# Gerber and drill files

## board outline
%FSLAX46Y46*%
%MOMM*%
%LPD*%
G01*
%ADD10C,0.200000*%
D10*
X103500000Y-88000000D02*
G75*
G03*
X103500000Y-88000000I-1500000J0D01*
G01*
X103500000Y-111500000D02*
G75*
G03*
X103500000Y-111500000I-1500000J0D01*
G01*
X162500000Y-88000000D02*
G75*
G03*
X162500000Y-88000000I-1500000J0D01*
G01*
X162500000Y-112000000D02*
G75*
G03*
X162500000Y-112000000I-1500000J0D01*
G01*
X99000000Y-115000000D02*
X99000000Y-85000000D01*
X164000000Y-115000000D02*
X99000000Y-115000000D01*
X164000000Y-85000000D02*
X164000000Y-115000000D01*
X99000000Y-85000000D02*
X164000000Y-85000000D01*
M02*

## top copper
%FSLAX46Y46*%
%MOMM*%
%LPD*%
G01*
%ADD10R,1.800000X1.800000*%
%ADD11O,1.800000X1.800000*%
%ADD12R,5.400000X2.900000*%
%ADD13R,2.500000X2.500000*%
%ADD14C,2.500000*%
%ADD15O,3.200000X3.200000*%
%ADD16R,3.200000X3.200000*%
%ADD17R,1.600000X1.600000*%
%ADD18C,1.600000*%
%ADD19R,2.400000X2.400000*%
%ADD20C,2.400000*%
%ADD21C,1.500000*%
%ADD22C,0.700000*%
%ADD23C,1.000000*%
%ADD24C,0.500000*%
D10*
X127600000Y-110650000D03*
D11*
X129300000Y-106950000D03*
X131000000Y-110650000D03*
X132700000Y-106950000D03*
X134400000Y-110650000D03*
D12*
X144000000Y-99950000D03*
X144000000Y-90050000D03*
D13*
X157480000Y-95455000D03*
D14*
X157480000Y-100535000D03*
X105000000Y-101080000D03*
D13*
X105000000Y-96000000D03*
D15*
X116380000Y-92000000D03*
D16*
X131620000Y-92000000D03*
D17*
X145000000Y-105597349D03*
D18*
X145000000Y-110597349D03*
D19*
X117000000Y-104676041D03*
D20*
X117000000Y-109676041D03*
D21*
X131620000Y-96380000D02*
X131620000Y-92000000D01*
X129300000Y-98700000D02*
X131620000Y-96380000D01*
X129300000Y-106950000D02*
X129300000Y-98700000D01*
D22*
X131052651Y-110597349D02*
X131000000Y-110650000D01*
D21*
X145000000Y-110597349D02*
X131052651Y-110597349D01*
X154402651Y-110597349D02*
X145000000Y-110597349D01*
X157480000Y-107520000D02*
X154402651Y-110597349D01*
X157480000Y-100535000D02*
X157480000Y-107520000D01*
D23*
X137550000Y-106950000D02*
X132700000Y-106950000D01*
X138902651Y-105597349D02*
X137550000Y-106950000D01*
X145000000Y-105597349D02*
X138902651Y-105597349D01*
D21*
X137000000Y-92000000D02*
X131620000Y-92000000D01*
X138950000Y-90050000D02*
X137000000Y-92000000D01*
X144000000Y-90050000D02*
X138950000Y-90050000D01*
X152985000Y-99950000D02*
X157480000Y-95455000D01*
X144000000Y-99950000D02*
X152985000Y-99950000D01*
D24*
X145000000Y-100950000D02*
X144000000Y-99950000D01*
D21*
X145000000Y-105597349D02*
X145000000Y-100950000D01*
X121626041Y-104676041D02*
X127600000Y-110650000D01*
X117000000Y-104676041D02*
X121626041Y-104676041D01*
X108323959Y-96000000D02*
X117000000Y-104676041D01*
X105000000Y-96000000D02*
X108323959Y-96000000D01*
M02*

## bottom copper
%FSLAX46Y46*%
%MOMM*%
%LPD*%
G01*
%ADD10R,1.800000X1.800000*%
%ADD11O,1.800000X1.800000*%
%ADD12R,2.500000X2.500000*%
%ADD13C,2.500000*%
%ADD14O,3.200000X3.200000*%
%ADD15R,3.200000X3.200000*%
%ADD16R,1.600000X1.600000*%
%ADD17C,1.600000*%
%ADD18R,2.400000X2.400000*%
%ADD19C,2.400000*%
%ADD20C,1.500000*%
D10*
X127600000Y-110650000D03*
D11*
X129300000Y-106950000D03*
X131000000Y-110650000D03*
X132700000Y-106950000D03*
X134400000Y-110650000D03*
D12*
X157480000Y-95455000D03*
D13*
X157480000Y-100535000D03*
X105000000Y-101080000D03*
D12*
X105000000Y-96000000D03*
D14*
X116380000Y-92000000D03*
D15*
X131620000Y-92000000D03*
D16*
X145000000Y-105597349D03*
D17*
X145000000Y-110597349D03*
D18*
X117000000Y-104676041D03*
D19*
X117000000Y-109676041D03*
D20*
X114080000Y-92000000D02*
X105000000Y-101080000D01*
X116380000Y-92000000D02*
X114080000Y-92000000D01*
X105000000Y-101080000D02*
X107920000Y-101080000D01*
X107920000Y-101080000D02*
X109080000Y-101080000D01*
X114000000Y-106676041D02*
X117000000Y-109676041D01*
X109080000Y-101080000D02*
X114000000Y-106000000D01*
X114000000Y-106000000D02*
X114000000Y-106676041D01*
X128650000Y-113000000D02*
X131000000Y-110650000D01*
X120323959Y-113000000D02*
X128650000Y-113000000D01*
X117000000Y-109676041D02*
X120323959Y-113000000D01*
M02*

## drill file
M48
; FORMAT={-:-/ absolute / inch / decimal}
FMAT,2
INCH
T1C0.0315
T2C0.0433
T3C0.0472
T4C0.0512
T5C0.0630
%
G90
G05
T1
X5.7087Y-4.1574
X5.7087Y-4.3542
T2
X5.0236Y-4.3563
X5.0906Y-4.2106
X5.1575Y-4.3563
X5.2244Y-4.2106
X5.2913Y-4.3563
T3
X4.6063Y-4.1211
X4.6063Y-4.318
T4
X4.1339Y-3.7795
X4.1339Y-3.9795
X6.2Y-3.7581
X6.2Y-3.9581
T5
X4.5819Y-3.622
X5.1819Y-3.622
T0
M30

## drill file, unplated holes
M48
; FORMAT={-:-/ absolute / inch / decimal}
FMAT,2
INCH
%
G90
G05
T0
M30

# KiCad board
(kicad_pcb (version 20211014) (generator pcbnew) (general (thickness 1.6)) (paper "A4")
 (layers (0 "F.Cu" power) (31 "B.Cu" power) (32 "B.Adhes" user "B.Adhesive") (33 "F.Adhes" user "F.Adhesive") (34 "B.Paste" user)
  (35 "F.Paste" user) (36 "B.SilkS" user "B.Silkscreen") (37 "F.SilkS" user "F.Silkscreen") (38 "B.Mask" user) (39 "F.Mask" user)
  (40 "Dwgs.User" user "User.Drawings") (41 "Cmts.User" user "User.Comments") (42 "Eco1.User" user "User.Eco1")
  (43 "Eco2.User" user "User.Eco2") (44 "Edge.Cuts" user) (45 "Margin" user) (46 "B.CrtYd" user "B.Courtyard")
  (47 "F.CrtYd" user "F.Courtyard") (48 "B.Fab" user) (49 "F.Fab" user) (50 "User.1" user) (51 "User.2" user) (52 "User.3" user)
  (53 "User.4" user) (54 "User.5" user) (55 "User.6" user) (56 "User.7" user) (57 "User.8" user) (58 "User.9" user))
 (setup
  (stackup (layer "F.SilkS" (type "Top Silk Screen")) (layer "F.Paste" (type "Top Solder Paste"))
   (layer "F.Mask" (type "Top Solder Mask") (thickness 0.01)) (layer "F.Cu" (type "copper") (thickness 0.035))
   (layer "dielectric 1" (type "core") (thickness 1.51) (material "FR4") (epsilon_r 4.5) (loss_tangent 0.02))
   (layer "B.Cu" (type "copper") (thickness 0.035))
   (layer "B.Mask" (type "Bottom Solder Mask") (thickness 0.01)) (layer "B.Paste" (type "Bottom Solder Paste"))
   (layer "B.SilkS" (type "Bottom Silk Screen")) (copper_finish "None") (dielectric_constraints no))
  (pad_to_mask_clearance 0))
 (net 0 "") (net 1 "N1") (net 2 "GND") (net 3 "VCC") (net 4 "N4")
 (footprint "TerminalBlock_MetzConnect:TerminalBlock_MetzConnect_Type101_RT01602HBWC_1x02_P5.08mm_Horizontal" (layer "F.Cu")
  (at 157.48 95.455 -90)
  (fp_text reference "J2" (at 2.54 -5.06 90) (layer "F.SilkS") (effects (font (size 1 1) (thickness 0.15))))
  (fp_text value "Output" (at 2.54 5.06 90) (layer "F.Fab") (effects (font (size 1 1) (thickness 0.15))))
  (pad "1" thru_hole rect (at 0 0 270) (size 2.5 2.5) (drill 1.3) (layers *.Cu *.Mask) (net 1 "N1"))
  (pad "2" thru_hole circle (at 5.08 0 270) (size 2.5 2.5) (drill 1.3) (layers *.Cu *.Mask) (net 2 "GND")))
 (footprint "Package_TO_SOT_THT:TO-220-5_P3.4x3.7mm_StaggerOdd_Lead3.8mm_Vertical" (layer "F.Cu") (at 127.6 110.65)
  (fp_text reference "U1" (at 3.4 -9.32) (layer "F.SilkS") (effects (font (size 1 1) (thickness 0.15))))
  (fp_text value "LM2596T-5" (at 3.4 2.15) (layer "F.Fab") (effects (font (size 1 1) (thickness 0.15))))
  (pad "1" thru_hole rect (at 0 0) (size 1.8 1.8) (drill 1.1) (layers *.Cu *.Mask) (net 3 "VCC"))
  (pad "2" thru_hole oval (at 1.7 -3.7) (size 1.8 1.8) (drill 1.1) (layers *.Cu *.Mask) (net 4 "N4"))
  (pad "3" thru_hole oval (at 3.4 0) (size 1.8 1.8) (drill 1.1) (layers *.Cu *.Mask) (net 2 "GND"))
  (pad "4" thru_hole oval (at 5.1 -3.7) (size 1.8 1.8) (drill 1.1) (layers *.Cu *.Mask) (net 1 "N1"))
  (pad "5" thru_hole oval (at 6.8 0) (size 1.8 1.8) (drill 1.1) (layers *.Cu *.Mask) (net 2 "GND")))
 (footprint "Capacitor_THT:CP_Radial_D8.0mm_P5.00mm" (layer "F.Cu") (at 145 105.597349 -90)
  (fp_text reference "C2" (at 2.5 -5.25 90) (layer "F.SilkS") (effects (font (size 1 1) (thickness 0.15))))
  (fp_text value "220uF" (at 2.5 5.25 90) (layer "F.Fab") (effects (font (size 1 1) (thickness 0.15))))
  (pad "1" thru_hole rect (at 0 0 270) (size 1.6 1.6) (drill 0.8) (layers *.Cu *.Mask) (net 1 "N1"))
  (pad "2" thru_hole circle (at 5 0 270) (size 1.6 1.6) (drill 0.8) (layers *.Cu *.Mask) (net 2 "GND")))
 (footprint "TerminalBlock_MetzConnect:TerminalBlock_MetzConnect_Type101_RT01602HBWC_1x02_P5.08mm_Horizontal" (layer "F.Cu") (at 105 96 -90)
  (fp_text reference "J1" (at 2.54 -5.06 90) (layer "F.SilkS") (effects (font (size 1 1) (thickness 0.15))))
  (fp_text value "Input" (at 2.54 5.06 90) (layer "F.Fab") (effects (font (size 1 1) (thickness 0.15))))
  (pad "1" thru_hole rect (at 0 0 270) (size 2.5 2.5) (drill 1.3) (layers *.Cu *.Mask) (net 3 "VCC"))
  (pad "2" thru_hole circle (at 5.08 0 270) (size 2.5 2.5) (drill 1.3) (layers *.Cu *.Mask) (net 2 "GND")))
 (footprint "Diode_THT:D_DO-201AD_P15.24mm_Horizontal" (layer "F.Cu") (at 131.62 92 180)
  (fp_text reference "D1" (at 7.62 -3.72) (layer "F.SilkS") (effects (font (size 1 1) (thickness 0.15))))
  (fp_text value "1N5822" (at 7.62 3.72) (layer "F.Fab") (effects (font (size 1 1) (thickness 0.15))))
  (pad "1" thru_hole rect (at 0 0 180) (size 3.2 3.2) (drill 1.6) (layers *.Cu *.Mask) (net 4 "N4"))
  (pad "2" thru_hole oval (at 15.24 0 180) (size 3.2 3.2) (drill 1.6) (layers *.Cu *.Mask) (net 2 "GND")))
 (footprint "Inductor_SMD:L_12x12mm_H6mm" (layer "F.Cu") (at 144 95 -90)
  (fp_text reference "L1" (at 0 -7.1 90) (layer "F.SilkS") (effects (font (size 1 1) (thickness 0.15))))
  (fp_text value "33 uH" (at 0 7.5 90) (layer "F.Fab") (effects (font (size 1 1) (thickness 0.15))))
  (pad "1" smd rect (at -4.95 0 270) (size 2.9 5.4) (layers "F.Cu" "F.Paste" "F.Mask") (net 4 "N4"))
  (pad "2" smd rect (at 4.95 0 270) (size 2.9 5.4) (layers "F.Cu" "F.Paste" "F.Mask") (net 1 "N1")))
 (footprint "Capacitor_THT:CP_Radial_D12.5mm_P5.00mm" (layer "F.Cu") (at 117 104.676041 -90)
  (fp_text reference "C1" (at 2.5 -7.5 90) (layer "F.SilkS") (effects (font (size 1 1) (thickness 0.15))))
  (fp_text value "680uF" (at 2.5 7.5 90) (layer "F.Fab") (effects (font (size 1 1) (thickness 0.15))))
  (pad "1" thru_hole rect (at 0 0 270) (size 2.4 2.4) (drill 1.2) (layers *.Cu *.Mask) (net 3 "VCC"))
  (pad "2" thru_hole circle (at 5 0 270) (size 2.4 2.4) (drill 1.2) (layers *.Cu *.Mask) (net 2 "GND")))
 (gr_circle (center 102 111.5) (end 103.5 111.5) (layer "Edge.Cuts") (width 0.2) (fill none))
 (gr_line (start 99 115) (end 99 85) (layer "Edge.Cuts") (width 0.2))
 (gr_circle (center 102 88) (end 103.5 88) (layer "Edge.Cuts") (width 0.2) (fill none))
 (gr_circle (center 161 88) (end 162.5 88) (layer "Edge.Cuts") (width 0.2) (fill none))
 (gr_line (start 164 115) (end 99 115) (layer "Edge.Cuts") (width 0.2))
 (gr_circle (center 161 112) (end 162.5 112) (layer "Edge.Cuts") (width 0.2) (fill none))
 (gr_line (start 164 85) (end 164 115) (layer "Edge.Cuts") (width 0.2))
 (gr_line (start 99 85) (end 164 85) (layer "Edge.Cuts") (width 0.2))
 (segment (start 108.323959 96) (end 117 104.676041) (width 1.5) (layer "F.Cu") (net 3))
 (segment (start 121.626041 104.676041) (end 127.6 110.65) (width 1.5) (layer "F.Cu") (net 3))
 (segment (start 117 104.676041) (end 121.626041 104.676041) (width 1.5) (layer "F.Cu") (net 3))
 (segment (start 105 96) (end 108.323959 96) (width 1.5) (layer "F.Cu") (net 3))
 (segment (start 145 110.597349) (end 131.052651 110.597349) (width 1.5) (layer "F.Cu") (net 2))
 (segment (start 157.48 107.52) (end 154.402651 110.597349) (width 1.5) (layer "F.Cu") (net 2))
 (segment (start 154.402651 110.597349) (end 145 110.597349) (width 1.5) (layer "F.Cu") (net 2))
 (segment (start 157.48 100.535) (end 157.48 107.52) (width 1.5) (layer "F.Cu") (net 2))
 (segment (start 131.052651 110.597349) (end 131 110.65) (width 0.7) (layer "F.Cu") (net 2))
 (segment (start 114 106) (end 114 106.676041) (width 1.5) (layer "B.Cu") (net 2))
 (segment (start 114 106.676041) (end 117 109.676041) (width 1.5) (layer "B.Cu") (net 2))
 (segment (start 117 109.676041) (end 120.323959 113) (width 1.5) (layer "B.Cu") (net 2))
 (segment (start 128.65 113) (end 131 110.65) (width 1.5) (layer "B.Cu") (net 2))
 (segment (start 107.92 101.08) (end 109.08 101.08) (width 1.5) (layer "B.Cu") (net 2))
 (segment (start 116.38 92) (end 114.08 92) (width 1.5) (layer "B.Cu") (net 2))
 (segment (start 114.08 92) (end 105 101.08) (width 1.5) (layer "B.Cu") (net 2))
 (segment (start 109.08 101.08) (end 114 106) (width 1.5) (layer "B.Cu") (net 2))
 (segment (start 105 101.08) (end 107.92 101.08) (width 1.5) (layer "B.Cu") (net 2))
 (segment (start 120.323959 113) (end 128.65 113) (width 1.5) (layer "B.Cu") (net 2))
 (segment (start 137.55 106.95) (end 132.7 106.95) (width 1) (layer "F.Cu") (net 1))
 (segment (start 145 105.597349) (end 138.902651 105.597349) (width 1) (layer "F.Cu") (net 1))
 (segment (start 152.985 99.95) (end 157.48 95.455) (width 1.5) (layer "F.Cu") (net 1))
 (segment (start 145 105.597349) (end 145 100.95) (width 1.5) (layer "F.Cu") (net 1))
 (segment (start 138.902651 105.597349) (end 137.55 106.95) (width 1) (layer "F.Cu") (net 1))
 (segment (start 144 99.95) (end 152.985 99.95) (width 1.5) (layer "F.Cu") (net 1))
 (segment (start 145 100.95) (end 144 99.95) (width 0.5) (layer "F.Cu") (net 1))
 (segment (start 144 90.05) (end 138.95 90.05) (width 1.5) (layer "F.Cu") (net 4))
 (segment (start 129.3 98.7) (end 131.62 96.38) (width 1.5) (layer "F.Cu") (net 4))
 (segment (start 137 92) (end 131.62 92) (width 1.5) (layer "F.Cu") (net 4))
 (segment (start 138.95 90.05) (end 137 92) (width 1.5) (layer "F.Cu") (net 4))
 (segment (start 129.3 106.95) (end 129.3 98.7) (width 1.5) (layer "F.Cu") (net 4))
 (segment (start 131.62 96.38) (end 131.62 92) (width 1.5) (layer "F.Cu") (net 4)))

